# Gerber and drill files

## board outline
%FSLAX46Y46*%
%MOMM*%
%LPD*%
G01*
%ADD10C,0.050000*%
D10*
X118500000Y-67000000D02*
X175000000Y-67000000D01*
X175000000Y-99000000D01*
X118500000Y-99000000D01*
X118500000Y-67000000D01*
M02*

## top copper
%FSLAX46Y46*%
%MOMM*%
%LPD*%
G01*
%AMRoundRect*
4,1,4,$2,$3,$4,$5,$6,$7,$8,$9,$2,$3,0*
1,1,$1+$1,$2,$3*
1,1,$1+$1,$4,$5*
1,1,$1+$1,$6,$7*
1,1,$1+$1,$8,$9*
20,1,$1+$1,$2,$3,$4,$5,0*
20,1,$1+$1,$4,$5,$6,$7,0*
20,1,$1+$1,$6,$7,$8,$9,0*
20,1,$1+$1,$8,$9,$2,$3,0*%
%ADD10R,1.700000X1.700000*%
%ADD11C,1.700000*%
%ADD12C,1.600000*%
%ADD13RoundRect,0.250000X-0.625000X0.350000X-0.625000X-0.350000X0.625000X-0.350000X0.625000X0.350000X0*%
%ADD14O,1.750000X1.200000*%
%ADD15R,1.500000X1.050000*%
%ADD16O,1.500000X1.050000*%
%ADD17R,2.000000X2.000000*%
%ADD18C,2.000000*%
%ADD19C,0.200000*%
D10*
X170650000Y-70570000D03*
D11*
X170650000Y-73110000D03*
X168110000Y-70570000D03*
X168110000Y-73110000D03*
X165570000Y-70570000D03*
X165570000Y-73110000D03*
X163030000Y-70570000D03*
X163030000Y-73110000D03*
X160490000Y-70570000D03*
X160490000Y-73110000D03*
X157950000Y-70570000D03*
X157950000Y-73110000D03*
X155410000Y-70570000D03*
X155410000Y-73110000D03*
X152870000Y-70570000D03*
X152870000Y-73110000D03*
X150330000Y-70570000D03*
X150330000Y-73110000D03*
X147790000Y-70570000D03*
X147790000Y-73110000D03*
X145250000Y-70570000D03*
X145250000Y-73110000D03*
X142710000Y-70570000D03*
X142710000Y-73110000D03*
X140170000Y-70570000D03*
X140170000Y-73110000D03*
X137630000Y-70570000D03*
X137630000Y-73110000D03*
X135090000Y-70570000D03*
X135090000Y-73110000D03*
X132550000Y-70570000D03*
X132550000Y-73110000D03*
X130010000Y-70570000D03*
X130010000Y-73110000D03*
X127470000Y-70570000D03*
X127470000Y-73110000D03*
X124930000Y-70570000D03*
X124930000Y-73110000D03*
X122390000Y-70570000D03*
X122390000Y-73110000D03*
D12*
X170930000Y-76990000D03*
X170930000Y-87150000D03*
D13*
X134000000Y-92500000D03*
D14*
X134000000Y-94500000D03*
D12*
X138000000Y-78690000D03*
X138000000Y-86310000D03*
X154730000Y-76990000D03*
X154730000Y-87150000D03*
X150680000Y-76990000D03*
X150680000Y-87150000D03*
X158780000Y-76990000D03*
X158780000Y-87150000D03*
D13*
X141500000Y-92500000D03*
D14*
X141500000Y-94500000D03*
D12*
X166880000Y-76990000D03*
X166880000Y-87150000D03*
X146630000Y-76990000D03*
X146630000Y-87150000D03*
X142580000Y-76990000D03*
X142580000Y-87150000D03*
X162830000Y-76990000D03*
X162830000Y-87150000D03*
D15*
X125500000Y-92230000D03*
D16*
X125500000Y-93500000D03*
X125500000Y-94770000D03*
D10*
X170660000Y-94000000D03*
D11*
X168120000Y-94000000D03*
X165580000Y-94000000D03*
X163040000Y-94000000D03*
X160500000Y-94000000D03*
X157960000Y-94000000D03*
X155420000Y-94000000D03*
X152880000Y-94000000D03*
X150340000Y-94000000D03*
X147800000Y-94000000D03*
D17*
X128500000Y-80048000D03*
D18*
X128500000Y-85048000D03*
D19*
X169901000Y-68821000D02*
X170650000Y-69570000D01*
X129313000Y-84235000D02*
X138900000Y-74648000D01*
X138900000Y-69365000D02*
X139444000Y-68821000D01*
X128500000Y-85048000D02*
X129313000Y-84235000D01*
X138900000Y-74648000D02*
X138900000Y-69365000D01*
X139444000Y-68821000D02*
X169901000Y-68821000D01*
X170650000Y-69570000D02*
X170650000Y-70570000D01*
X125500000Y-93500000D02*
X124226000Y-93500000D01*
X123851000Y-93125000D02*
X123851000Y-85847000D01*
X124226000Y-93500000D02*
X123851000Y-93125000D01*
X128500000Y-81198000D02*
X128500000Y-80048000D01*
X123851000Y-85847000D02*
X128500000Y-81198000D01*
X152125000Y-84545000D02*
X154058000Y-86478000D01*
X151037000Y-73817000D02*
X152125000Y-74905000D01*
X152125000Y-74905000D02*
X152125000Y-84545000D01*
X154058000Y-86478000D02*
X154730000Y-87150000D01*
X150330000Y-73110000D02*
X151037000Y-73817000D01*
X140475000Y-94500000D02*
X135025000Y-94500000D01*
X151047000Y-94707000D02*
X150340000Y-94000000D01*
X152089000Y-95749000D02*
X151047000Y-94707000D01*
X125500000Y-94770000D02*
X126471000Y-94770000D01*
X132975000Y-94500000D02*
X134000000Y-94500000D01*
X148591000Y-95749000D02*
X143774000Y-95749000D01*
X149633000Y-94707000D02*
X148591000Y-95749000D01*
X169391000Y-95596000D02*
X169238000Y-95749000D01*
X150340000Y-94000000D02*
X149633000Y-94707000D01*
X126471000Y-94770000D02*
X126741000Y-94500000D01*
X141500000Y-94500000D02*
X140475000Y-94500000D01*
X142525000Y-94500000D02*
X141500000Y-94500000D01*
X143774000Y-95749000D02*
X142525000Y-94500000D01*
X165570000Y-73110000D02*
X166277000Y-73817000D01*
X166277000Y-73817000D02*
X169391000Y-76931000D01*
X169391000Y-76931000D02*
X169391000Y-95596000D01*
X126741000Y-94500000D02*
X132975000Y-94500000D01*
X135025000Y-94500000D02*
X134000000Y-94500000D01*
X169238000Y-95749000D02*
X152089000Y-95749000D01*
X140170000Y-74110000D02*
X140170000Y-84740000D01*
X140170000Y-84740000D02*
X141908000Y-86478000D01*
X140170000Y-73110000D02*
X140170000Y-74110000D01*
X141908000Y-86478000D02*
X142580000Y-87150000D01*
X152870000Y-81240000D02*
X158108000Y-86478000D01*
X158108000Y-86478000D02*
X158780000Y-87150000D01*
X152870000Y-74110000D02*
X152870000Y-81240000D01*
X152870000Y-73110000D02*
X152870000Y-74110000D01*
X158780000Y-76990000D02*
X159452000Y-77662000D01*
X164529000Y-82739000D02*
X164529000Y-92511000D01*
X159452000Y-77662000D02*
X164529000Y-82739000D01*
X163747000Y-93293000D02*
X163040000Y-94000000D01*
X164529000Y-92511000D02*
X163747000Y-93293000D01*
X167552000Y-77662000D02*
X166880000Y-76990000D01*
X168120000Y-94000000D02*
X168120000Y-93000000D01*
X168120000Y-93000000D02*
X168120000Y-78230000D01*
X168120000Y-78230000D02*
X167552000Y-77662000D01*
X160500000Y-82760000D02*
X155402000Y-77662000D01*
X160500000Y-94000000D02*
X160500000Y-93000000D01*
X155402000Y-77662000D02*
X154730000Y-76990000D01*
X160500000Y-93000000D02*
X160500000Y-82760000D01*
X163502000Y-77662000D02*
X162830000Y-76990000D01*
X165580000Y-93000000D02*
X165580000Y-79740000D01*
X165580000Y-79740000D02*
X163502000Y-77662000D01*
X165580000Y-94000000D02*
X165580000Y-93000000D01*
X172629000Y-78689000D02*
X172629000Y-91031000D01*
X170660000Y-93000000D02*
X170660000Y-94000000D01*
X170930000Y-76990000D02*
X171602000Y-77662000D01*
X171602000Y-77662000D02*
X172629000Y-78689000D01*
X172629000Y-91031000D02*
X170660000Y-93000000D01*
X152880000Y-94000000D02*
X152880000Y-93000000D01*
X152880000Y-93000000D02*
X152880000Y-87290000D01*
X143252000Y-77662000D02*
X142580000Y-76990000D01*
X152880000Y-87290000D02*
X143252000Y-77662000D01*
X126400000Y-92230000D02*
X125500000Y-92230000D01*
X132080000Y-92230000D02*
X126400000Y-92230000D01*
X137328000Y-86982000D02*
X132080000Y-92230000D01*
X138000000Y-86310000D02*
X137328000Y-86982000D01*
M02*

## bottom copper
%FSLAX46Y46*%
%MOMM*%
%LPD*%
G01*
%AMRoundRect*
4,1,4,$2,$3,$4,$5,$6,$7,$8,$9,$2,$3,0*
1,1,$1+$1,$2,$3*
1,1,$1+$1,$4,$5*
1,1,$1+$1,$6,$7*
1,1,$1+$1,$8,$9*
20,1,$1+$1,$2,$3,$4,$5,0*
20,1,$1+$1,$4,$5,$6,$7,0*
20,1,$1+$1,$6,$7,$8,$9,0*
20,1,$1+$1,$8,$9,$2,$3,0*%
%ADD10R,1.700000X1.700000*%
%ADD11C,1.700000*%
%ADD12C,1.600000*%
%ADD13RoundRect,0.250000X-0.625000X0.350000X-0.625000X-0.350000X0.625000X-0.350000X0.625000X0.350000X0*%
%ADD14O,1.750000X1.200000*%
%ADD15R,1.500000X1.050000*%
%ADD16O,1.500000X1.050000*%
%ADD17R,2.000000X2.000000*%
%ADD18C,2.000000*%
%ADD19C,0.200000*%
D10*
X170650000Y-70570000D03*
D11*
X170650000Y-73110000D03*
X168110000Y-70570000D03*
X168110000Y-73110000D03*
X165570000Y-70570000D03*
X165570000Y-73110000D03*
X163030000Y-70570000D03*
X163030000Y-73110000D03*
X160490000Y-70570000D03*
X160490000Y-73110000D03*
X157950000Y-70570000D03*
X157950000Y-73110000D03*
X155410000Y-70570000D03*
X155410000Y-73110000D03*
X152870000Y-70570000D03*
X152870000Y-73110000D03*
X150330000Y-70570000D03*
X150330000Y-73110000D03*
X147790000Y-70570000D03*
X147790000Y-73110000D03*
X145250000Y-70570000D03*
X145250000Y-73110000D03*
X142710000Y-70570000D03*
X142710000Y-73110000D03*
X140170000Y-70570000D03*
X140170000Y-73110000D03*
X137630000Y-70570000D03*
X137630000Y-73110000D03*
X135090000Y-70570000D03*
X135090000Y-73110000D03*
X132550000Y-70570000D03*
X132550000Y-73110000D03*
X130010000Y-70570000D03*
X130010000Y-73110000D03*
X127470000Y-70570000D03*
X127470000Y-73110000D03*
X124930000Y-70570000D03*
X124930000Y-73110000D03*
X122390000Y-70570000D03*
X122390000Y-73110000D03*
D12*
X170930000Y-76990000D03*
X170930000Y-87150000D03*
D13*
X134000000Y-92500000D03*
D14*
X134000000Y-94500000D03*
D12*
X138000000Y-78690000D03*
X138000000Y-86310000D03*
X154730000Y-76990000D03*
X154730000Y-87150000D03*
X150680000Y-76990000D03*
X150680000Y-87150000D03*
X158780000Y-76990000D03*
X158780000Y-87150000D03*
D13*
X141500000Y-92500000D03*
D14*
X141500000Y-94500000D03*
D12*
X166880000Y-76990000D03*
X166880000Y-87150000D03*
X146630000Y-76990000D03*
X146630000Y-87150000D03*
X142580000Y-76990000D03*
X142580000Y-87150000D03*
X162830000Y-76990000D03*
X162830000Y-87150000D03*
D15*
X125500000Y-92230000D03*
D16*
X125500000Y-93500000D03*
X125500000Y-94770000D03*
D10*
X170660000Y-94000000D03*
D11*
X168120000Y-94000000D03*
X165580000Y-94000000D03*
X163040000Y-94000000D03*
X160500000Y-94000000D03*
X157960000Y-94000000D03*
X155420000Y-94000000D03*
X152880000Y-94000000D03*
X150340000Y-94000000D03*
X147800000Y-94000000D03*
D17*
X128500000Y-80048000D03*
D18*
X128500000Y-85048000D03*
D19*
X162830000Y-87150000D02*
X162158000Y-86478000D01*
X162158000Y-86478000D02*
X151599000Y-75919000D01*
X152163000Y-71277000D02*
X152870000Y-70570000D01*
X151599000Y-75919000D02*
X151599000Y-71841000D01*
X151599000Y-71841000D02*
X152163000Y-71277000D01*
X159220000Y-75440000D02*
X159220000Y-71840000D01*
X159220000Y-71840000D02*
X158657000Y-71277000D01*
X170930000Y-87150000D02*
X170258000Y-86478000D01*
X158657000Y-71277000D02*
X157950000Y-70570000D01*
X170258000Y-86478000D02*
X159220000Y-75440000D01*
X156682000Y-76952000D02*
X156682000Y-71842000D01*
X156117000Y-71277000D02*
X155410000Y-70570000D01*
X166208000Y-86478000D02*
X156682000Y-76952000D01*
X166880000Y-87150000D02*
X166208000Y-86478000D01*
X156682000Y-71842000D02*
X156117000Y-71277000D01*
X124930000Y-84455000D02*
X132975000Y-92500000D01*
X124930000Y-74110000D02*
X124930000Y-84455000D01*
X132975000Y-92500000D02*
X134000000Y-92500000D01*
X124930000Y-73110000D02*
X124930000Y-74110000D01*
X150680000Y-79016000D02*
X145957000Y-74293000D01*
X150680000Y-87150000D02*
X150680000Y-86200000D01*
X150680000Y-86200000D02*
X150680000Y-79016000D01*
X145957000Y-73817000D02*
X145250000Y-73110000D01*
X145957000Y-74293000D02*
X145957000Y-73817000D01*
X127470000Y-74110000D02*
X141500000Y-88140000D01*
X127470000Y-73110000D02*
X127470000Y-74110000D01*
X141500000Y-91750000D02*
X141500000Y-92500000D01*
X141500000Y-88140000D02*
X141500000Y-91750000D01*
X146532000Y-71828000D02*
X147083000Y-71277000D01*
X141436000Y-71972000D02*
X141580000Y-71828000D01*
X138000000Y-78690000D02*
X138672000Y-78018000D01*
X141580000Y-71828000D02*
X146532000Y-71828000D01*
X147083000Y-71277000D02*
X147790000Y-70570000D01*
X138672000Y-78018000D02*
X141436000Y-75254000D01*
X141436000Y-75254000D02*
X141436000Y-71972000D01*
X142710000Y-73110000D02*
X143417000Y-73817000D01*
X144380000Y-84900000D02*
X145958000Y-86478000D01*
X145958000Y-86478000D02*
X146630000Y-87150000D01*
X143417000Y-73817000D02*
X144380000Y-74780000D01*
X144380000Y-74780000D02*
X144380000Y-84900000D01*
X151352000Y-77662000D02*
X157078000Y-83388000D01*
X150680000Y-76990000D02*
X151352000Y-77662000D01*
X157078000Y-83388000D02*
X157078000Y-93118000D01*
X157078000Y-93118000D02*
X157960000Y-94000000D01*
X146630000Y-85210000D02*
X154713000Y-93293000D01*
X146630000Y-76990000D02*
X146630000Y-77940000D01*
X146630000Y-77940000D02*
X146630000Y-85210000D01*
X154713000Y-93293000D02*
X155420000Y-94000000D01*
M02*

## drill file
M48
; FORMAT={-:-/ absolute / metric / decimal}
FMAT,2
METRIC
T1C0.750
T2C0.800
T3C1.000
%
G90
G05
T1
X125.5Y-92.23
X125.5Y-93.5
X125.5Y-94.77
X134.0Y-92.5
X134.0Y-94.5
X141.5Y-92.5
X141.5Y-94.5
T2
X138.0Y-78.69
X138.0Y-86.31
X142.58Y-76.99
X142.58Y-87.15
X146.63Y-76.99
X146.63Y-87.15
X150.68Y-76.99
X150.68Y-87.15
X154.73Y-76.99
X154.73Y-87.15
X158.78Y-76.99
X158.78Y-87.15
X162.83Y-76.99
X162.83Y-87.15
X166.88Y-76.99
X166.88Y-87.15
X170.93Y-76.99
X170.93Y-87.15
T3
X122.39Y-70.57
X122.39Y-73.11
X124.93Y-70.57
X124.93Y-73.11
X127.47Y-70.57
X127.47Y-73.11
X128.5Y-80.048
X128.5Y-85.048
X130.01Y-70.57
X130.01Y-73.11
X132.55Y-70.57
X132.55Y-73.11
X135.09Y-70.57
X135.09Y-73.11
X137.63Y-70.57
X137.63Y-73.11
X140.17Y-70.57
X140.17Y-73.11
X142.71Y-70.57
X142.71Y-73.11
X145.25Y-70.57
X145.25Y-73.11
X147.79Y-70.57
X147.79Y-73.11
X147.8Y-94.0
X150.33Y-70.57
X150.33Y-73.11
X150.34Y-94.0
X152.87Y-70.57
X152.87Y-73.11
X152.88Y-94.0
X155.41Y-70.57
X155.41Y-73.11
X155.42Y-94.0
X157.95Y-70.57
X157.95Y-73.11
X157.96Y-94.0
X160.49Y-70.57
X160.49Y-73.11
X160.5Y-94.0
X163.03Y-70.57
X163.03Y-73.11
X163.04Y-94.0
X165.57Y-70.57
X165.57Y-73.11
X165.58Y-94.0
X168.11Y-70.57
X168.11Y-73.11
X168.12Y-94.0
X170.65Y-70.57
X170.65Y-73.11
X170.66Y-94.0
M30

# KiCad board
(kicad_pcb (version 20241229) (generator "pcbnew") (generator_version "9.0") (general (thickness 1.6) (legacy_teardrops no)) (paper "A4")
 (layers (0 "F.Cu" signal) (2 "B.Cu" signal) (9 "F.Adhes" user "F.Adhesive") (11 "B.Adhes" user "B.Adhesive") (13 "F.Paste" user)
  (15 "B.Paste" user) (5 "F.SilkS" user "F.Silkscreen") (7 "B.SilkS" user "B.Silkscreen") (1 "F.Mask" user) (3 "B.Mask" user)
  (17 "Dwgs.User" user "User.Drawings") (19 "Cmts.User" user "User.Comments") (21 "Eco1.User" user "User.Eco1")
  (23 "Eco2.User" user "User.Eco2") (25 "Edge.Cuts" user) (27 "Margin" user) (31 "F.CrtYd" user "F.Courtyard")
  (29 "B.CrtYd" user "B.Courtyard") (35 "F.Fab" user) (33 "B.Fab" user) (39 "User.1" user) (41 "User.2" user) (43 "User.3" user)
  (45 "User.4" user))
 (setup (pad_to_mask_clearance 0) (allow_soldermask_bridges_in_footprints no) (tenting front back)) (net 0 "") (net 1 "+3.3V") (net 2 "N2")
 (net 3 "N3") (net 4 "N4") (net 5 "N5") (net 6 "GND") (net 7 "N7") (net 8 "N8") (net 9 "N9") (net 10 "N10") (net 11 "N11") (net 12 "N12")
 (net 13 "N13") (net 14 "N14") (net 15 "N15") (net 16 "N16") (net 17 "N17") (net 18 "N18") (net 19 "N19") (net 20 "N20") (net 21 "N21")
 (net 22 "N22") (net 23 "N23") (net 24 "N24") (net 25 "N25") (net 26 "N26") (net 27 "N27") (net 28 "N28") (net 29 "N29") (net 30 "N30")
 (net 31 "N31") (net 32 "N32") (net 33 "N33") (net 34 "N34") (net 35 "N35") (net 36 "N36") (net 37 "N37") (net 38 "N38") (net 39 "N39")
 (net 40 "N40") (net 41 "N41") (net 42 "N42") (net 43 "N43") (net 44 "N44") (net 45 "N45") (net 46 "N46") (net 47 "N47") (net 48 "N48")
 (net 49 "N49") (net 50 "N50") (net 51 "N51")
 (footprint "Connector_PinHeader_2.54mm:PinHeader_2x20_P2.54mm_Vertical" (layer "F.Cu") (at 170.65 70.57 -90)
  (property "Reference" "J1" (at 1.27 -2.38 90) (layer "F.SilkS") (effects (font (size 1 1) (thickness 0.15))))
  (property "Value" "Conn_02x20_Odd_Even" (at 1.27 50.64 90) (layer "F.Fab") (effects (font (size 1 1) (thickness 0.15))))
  (pad "1" thru_hole rect (at 0 0 270) (size 1.7 1.7) (drill 1) (layers "*.Cu" "*.Mask") (remove_unused_layers no) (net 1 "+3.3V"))
  (pad "2" thru_hole circle (at 2.54 0 270) (size 1.7 1.7) (drill 1) (layers "*.Cu" "*.Mask") (remove_unused_layers no) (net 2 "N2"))
  (pad "3" thru_hole circle (at 0 2.54 270) (size 1.7 1.7) (drill 1) (layers "*.Cu" "*.Mask") (remove_unused_layers no) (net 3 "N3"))
  (pad "4" thru_hole circle (at 2.54 2.54 270) (size 1.7 1.7) (drill 1) (layers "*.Cu" "*.Mask") (remove_unused_layers no) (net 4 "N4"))
  (pad "5" thru_hole circle (at 0 5.08 270) (size 1.7 1.7) (drill 1) (layers "*.Cu" "*.Mask") (remove_unused_layers no) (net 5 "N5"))
  (pad "6" thru_hole circle (at 2.54 5.08 270) (size 1.7 1.7) (drill 1) (layers "*.Cu" "*.Mask") (remove_unused_layers no) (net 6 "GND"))
  (pad "7" thru_hole circle (at 0 7.62 270) (size 1.7 1.7) (drill 1) (layers "*.Cu" "*.Mask") (remove_unused_layers no) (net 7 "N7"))
  (pad "8" thru_hole circle (at 2.54 7.62 270) (size 1.7 1.7) (drill 1) (layers "*.Cu" "*.Mask") (remove_unused_layers no) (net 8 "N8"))
  (pad "9" thru_hole circle (at 0 10.16 270) (size 1.7 1.7) (drill 1) (layers "*.Cu" "*.Mask") (remove_unused_layers no) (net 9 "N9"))
  (pad "10" thru_hole circle (at 2.54 10.16 270) (size 1.7 1.7) (drill 1) (layers "*.Cu" "*.Mask") (remove_unused_layers no) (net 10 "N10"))
  (pad "11" thru_hole circle (at 0 12.7 270) (size 1.7 1.7) (drill 1) (layers "*.Cu" "*.Mask") (remove_unused_layers no) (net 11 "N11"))
  (pad "12" thru_hole circle (at 2.54 12.7 270) (size 1.7 1.7) (drill 1) (layers "*.Cu" "*.Mask") (remove_unused_layers no) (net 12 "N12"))
  (pad "13" thru_hole circle (at 0 15.24 270) (size 1.7 1.7) (drill 1) (layers "*.Cu" "*.Mask") (remove_unused_layers no) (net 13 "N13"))
  (pad "14" thru_hole circle (at 2.54 15.24 270) (size 1.7 1.7) (drill 1) (layers "*.Cu" "*.Mask") (remove_unused_layers no) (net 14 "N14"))
  (pad "15" thru_hole circle (at 0 17.78 270) (size 1.7 1.7) (drill 1) (layers "*.Cu" "*.Mask") (remove_unused_layers no) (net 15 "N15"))
  (pad "16" thru_hole circle (at 2.54 17.78 270) (size 1.7 1.7) (drill 1) (layers "*.Cu" "*.Mask") (remove_unused_layers no) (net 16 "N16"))
  (pad "17" thru_hole circle (at 0 20.32 270) (size 1.7 1.7) (drill 1) (layers "*.Cu" "*.Mask") (remove_unused_layers no) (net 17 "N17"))
  (pad "18" thru_hole circle (at 2.54 20.32 270) (size 1.7 1.7) (drill 1) (layers "*.Cu" "*.Mask") (remove_unused_layers no) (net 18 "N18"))
  (pad "19" thru_hole circle (at 0 22.86 270) (size 1.7 1.7) (drill 1) (layers "*.Cu" "*.Mask") (remove_unused_layers no) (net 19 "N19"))
  (pad "20" thru_hole circle (at 2.54 22.86 270) (size 1.7 1.7) (drill 1) (layers "*.Cu" "*.Mask") (remove_unused_layers no) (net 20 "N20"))
  (pad "21" thru_hole circle (at 0 25.4 270) (size 1.7 1.7) (drill 1) (layers "*.Cu" "*.Mask") (remove_unused_layers no) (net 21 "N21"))
  (pad "22" thru_hole circle (at 2.54 25.4 270) (size 1.7 1.7) (drill 1) (layers "*.Cu" "*.Mask") (remove_unused_layers no) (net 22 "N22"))
  (pad "23" thru_hole circle (at 0 27.94 270) (size 1.7 1.7) (drill 1) (layers "*.Cu" "*.Mask") (remove_unused_layers no) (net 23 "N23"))
  (pad "24" thru_hole circle (at 2.54 27.94 270) (size 1.7 1.7) (drill 1) (layers "*.Cu" "*.Mask") (remove_unused_layers no) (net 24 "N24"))
  (pad "25" thru_hole circle (at 0 30.48 270) (size 1.7 1.7) (drill 1) (layers "*.Cu" "*.Mask") (remove_unused_layers no) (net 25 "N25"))
  (pad "26" thru_hole circle (at 2.54 30.48 270) (size 1.7 1.7) (drill 1) (layers "*.Cu" "*.Mask") (remove_unused_layers no) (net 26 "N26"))
  (pad "27" thru_hole circle (at 0 33.02 270) (size 1.7 1.7) (drill 1) (layers "*.Cu" "*.Mask") (remove_unused_layers no) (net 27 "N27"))
  (pad "28" thru_hole circle (at 2.54 33.02 270) (size 1.7 1.7) (drill 1) (layers "*.Cu" "*.Mask") (remove_unused_layers no) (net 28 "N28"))
  (pad "29" thru_hole circle (at 0 35.56 270) (size 1.7 1.7) (drill 1) (layers "*.Cu" "*.Mask") (remove_unused_layers no) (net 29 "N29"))
  (pad "30" thru_hole circle (at 2.54 35.56 270) (size 1.7 1.7) (drill 1) (layers "*.Cu" "*.Mask") (remove_unused_layers no) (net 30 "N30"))
  (pad "31" thru_hole circle (at 0 38.1 270) (size 1.7 1.7) (drill 1) (layers "*.Cu" "*.Mask") (remove_unused_layers no) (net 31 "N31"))
  (pad "32" thru_hole circle (at 2.54 38.1 270) (size 1.7 1.7) (drill 1) (layers "*.Cu" "*.Mask") (remove_unused_layers no) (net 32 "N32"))
  (pad "33" thru_hole circle (at 0 40.64 270) (size 1.7 1.7) (drill 1) (layers "*.Cu" "*.Mask") (remove_unused_layers no) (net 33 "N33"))
  (pad "34" thru_hole circle (at 2.54 40.64 270) (size 1.7 1.7) (drill 1) (layers "*.Cu" "*.Mask") (remove_unused_layers no) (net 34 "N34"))
  (pad "35" thru_hole circle (at 0 43.18 270) (size 1.7 1.7) (drill 1) (layers "*.Cu" "*.Mask") (remove_unused_layers no) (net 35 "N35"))
  (pad "36" thru_hole circle (at 2.54 43.18 270) (size 1.7 1.7) (drill 1) (layers "*.Cu" "*.Mask") (remove_unused_layers no) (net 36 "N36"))
  (pad "37" thru_hole circle (at 0 45.72 270) (size 1.7 1.7) (drill 1) (layers "*.Cu" "*.Mask") (remove_unused_layers no) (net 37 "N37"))
  (pad "38" thru_hole circle (at 2.54 45.72 270) (size 1.7 1.7) (drill 1) (layers "*.Cu" "*.Mask") (remove_unused_layers no) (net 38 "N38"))
  (pad "39" thru_hole circle (at 0 48.26 270) (size 1.7 1.7) (drill 1) (layers "*.Cu" "*.Mask") (remove_unused_layers no) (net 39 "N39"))
  (pad "40" thru_hole circle (at 2.54 48.26 270) (size 1.7 1.7) (drill 1) (layers "*.Cu" "*.Mask") (remove_unused_layers no) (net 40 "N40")))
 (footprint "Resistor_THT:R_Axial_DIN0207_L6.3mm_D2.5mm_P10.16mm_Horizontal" (layer "F.Cu") (at 170.93 76.99 -90)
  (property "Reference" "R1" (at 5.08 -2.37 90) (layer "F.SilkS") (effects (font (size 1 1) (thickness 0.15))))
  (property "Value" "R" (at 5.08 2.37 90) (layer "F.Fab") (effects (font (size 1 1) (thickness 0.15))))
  (pad "1" thru_hole circle (at 0 0 270) (size 1.6 1.6) (drill 0.8) (layers "*.Cu" "*.Mask") (remove_unused_layers no) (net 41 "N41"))
  (pad "2" thru_hole circle (at 10.16 0 270) (size 1.6 1.6) (drill 0.8) (layers "*.Cu" "*.Mask") (remove_unused_layers no) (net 11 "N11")))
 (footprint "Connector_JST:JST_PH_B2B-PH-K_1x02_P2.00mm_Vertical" (layer "F.Cu") (at 134 92.5 -90)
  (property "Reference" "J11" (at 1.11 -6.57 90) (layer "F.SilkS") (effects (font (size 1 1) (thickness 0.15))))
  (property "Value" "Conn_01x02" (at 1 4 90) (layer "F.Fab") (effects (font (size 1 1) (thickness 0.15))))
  (pad "1" thru_hole roundrect (at 0 0 270) (size 1.2 1.75) (drill 0.75) (layers "*.Cu" "*.Mask") (remove_unused_layers no)
   (roundrect_rratio 0.208333) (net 38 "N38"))
  (pad "2" thru_hole oval (at 2 0 270) (size 1.2 1.75) (drill 0.75) (layers "*.Cu" "*.Mask") (remove_unused_layers no) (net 6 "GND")))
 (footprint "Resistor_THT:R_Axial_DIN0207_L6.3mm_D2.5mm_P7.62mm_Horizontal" (layer "F.Cu") (at 138 78.69 -90)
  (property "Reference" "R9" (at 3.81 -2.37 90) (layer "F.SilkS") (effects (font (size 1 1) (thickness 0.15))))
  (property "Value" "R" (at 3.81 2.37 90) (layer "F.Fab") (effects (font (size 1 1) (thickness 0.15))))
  (pad "1" thru_hole circle (at 0 0 270) (size 1.6 1.6) (drill 0.8) (layers "*.Cu" "*.Mask") (remove_unused_layers no) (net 19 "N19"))
  (pad "2" thru_hole circle (at 7.62 0 270) (size 1.6 1.6) (drill 0.8) (layers "*.Cu" "*.Mask") (remove_unused_layers no) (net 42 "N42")))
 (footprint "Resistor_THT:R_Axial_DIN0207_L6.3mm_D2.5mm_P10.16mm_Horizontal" (layer "F.Cu") (at 154.73 76.99 -90)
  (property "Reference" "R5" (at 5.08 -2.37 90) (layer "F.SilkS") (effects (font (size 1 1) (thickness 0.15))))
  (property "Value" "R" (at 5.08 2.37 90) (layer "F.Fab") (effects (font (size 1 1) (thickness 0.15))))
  (pad "1" thru_hole circle (at 0 0 270) (size 1.6 1.6) (drill 0.8) (layers "*.Cu" "*.Mask") (remove_unused_layers no) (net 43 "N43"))
  (pad "2" thru_hole circle (at 10.16 0 270) (size 1.6 1.6) (drill 0.8) (layers "*.Cu" "*.Mask") (remove_unused_layers no) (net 18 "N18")))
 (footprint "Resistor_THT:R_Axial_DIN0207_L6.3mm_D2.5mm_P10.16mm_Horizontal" (layer "F.Cu") (at 150.68 76.99 -90)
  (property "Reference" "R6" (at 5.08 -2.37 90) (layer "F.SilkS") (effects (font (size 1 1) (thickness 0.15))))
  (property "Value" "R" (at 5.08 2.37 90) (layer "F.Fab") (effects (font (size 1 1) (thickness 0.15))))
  (pad "1" thru_hole circle (at 0 0 270) (size 1.6 1.6) (drill 0.8) (layers "*.Cu" "*.Mask") (remove_unused_layers no) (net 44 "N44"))
  (pad "2" thru_hole circle (at 10.16 0 270) (size 1.6 1.6) (drill 0.8) (layers "*.Cu" "*.Mask") (remove_unused_layers no) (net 22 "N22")))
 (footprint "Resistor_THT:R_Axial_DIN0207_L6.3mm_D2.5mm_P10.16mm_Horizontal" (layer "F.Cu") (at 158.78 76.99 -90)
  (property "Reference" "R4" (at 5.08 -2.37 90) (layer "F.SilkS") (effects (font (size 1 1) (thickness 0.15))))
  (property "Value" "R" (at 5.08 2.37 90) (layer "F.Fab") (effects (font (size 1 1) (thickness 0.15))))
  (pad "1" thru_hole circle (at 0 0 270) (size 1.6 1.6) (drill 0.8) (layers "*.Cu" "*.Mask") (remove_unused_layers no) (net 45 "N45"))
  (pad "2" thru_hole circle (at 10.16 0 270) (size 1.6 1.6) (drill 0.8) (layers "*.Cu" "*.Mask") (remove_unused_layers no) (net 16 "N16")))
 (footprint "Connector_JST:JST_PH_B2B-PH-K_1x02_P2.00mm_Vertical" (layer "F.Cu") (at 141.5 92.5 -90)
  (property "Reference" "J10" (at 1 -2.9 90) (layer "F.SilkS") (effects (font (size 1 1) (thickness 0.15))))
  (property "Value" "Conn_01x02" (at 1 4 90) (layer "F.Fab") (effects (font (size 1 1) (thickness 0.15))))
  (pad "1" thru_hole roundrect (at 0 0 270) (size 1.2 1.75) (drill 0.75) (layers "*.Cu" "*.Mask") (remove_unused_layers no)
   (roundrect_rratio 0.208333) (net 36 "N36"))
  (pad "2" thru_hole oval (at 2 0 270) (size 1.2 1.75) (drill 0.75) (layers "*.Cu" "*.Mask") (remove_unused_layers no) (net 6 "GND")))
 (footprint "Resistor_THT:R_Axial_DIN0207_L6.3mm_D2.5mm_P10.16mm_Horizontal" (layer "F.Cu") (at 166.88 76.99 -90)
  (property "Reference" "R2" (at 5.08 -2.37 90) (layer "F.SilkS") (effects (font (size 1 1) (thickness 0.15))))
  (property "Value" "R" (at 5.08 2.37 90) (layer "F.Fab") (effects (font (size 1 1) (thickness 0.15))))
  (pad "1" thru_hole circle (at 0 0 270) (size 1.6 1.6) (drill 0.8) (layers "*.Cu" "*.Mask") (remove_unused_layers no) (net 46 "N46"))
  (pad "2" thru_hole circle (at 10.16 0 270) (size 1.6 1.6) (drill 0.8) (layers "*.Cu" "*.Mask") (remove_unused_layers no) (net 13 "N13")))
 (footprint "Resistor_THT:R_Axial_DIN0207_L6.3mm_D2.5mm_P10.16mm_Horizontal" (layer "F.Cu") (at 146.63 76.99 -90)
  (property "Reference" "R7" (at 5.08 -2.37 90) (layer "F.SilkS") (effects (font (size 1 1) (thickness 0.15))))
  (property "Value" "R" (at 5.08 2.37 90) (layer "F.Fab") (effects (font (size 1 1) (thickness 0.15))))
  (pad "1" thru_hole circle (at 0 0 270) (size 1.6 1.6) (drill 0.8) (layers "*.Cu" "*.Mask") (remove_unused_layers no) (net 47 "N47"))
  (pad "2" thru_hole circle (at 10.16 0 270) (size 1.6 1.6) (drill 0.8) (layers "*.Cu" "*.Mask") (remove_unused_layers no) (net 24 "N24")))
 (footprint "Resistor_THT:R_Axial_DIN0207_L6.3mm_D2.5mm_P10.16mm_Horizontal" (layer "F.Cu") (at 142.58 76.99 -90)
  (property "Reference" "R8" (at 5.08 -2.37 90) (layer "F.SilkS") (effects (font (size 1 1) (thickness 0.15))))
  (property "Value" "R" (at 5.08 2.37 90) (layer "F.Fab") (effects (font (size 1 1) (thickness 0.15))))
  (pad "1" thru_hole circle (at 0 0 270) (size 1.6 1.6) (drill 0.8) (layers "*.Cu" "*.Mask") (remove_unused_layers no) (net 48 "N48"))
  (pad "2" thru_hole circle (at 10.16 0 270) (size 1.6 1.6) (drill 0.8) (layers "*.Cu" "*.Mask") (remove_unused_layers no) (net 26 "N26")))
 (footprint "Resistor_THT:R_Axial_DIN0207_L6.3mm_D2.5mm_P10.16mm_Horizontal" (layer "F.Cu") (at 162.83 76.99 -90)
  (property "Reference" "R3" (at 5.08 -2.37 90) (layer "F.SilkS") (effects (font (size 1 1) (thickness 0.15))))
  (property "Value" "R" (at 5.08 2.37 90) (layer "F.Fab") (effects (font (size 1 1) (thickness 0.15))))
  (pad "1" thru_hole circle (at 0 0 270) (size 1.6 1.6) (drill 0.8) (layers "*.Cu" "*.Mask") (remove_unused_layers no) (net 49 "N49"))
  (pad "2" thru_hole circle (at 10.16 0 270) (size 1.6 1.6) (drill 0.8) (layers "*.Cu" "*.Mask") (remove_unused_layers no) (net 15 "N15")))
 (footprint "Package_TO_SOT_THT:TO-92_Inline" (layer "F.Cu") (at 125.5 92.23 -90)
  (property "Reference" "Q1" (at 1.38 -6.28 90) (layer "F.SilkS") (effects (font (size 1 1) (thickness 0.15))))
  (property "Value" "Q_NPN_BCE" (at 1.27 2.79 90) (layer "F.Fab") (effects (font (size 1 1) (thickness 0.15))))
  (pad "1" thru_hole rect (at 0 0 270) (size 1.05 1.5) (drill 0.75) (layers "*.Cu" "*.Mask") (remove_unused_layers no) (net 42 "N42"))
  (pad "2" thru_hole oval (at 1.27 0 270) (size 1.05 1.5) (drill 0.75) (layers "*.Cu" "*.Mask") (remove_unused_layers no) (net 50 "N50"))
  (pad "3" thru_hole oval (at 2.54 0 270) (size 1.05 1.5) (drill 0.75) (layers "*.Cu" "*.Mask") (remove_unused_layers no) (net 6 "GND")))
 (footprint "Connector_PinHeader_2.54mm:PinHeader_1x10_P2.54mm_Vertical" (layer "F.Cu") (at 170.66 94 -90)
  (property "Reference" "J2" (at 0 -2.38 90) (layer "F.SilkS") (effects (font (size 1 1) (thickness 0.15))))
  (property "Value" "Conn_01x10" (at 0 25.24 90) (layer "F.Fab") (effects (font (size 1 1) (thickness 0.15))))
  (pad "1" thru_hole rect (at 0 0 270) (size 1.7 1.7) (drill 1) (layers "*.Cu" "*.Mask") (remove_unused_layers no) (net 41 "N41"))
  (pad "2" thru_hole circle (at 0 2.54 270) (size 1.7 1.7) (drill 1) (layers "*.Cu" "*.Mask") (remove_unused_layers no) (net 46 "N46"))
  (pad "3" thru_hole circle (at 0 5.08 270) (size 1.7 1.7) (drill 1) (layers "*.Cu" "*.Mask") (remove_unused_layers no) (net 49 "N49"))
  (pad "4" thru_hole circle (at 0 7.62 270) (size 1.7 1.7) (drill 1) (layers "*.Cu" "*.Mask") (remove_unused_layers no) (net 45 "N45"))
  (pad "5" thru_hole circle (at 0 10.16 270) (size 1.7 1.7) (drill 1) (layers "*.Cu" "*.Mask") (remove_unused_layers no) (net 43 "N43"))
  (pad "6" thru_hole circle (at 0 12.7 270) (size 1.7 1.7) (drill 1) (layers "*.Cu" "*.Mask") (remove_unused_layers no) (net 44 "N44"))
  (pad "7" thru_hole circle (at 0 15.24 270) (size 1.7 1.7) (drill 1) (layers "*.Cu" "*.Mask") (remove_unused_layers no) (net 47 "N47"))
  (pad "8" thru_hole circle (at 0 17.78 270) (size 1.7 1.7) (drill 1) (layers "*.Cu" "*.Mask") (remove_unused_layers no) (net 48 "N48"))
  (pad "9" thru_hole circle (at 0 20.32 270) (size 1.7 1.7) (drill 1) (layers "*.Cu" "*.Mask") (remove_unused_layers no) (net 6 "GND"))
  (pad "10" thru_hole circle (at 0 22.86 270) (size 1.7 1.7) (drill 1) (layers "*.Cu" "*.Mask") (remove_unused_layers no) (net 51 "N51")))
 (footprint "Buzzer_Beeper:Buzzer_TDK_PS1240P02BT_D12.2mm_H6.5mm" (layer "F.Cu") (at 128.5 80.048 -90)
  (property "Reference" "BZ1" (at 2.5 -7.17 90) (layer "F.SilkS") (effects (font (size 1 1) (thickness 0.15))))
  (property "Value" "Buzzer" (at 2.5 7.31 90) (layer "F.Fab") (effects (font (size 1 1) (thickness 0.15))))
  (pad "1" thru_hole rect (at 0 0 270) (size 2 2) (drill 1) (layers "*.Cu" "*.Mask") (remove_unused_layers no) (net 50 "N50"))
  (pad "2" thru_hole circle (at 5 0 270) (size 2 2) (drill 1) (layers "*.Cu" "*.Mask") (remove_unused_layers no) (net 1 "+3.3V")))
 (gr_rect (start 118.5 67) (end 175 99) (stroke (width 0.05) (type default)) (fill no) (layer "Edge.Cuts"))
 (segment (start 169.901 68.821) (end 170.65 69.57) (width 0.2) (layer "F.Cu") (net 1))
 (segment (start 129.313 84.235) (end 138.9 74.648) (width 0.2) (layer "F.Cu") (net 1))
 (segment (start 138.9 69.365) (end 139.444 68.821) (width 0.2) (layer "F.Cu") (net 1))
 (segment (start 128.5 85.048) (end 129.313 84.235) (width 0.2) (layer "F.Cu") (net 1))
 (segment (start 138.9 74.648) (end 138.9 69.365) (width 0.2) (layer "F.Cu") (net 1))
 (segment (start 139.444 68.821) (end 169.901 68.821) (width 0.2) (layer "F.Cu") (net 1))
 (segment (start 170.65 69.57) (end 170.65 70.57) (width 0.2) (layer "F.Cu") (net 1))
 (segment (start 125.5 93.5) (end 124.226 93.5) (width 0.2) (layer "F.Cu") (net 50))
 (segment (start 123.851 93.125) (end 123.851 85.847) (width 0.2) (layer "F.Cu") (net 50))
 (segment (start 124.226 93.5) (end 123.851 93.125) (width 0.2) (layer "F.Cu") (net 50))
 (segment (start 128.5 81.198) (end 128.5 80.048) (width 0.2) (layer "F.Cu") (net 50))
 (segment (start 123.851 85.847) (end 128.5 81.198) (width 0.2) (layer "F.Cu") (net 50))
 (segment (start 152.125 84.545) (end 154.058 86.478) (width 0.2) (layer "F.Cu") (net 18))
 (segment (start 151.037 73.817) (end 152.125 74.905) (width 0.2) (layer "F.Cu") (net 18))
 (segment (start 152.125 74.905) (end 152.125 84.545) (width 0.2) (layer "F.Cu") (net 18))
 (segment (start 154.058 86.478) (end 154.73 87.15) (width 0.2) (layer "F.Cu") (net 18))
 (segment (start 150.33 73.11) (end 151.037 73.817) (width 0.2) (layer "F.Cu") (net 18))
 (segment (start 162.83 87.15) (end 162.158 86.478) (width 0.2) (layer "B.Cu") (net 15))
 (segment (start 162.158 86.478) (end 151.599 75.919) (width 0.2) (layer "B.Cu") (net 15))
 (segment (start 152.163 71.277) (end 152.87 70.57) (width 0.2) (layer "B.Cu") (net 15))
 (segment (start 151.599 75.919) (end 151.599 71.841) (width 0.2) (layer "B.Cu") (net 15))
 (segment (start 151.599 71.841) (end 152.163 71.277) (width 0.2) (layer "B.Cu") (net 15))
 (segment (start 159.22 75.44) (end 159.22 71.84) (width 0.2) (layer "B.Cu") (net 11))
 (segment (start 159.22 71.84) (end 158.657 71.277) (width 0.2) (layer "B.Cu") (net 11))
 (segment (start 170.93 87.15) (end 170.258 86.478) (width 0.2) (layer "B.Cu") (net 11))
 (segment (start 158.657 71.277) (end 157.95 70.57) (width 0.2) (layer "B.Cu") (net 11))
 (segment (start 170.258 86.478) (end 159.22 75.44) (width 0.2) (layer "B.Cu") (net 11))
 (segment (start 156.682 76.952) (end 156.682 71.842) (width 0.2) (layer "B.Cu") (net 13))
 (segment (start 156.117 71.277) (end 155.41 70.57) (width 0.2) (layer "B.Cu") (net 13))
 (segment (start 166.208 86.478) (end 156.682 76.952) (width 0.2) (layer "B.Cu") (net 13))
 (segment (start 166.88 87.15) (end 166.208 86.478) (width 0.2) (layer "B.Cu") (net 13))
 (segment (start 156.682 71.842) (end 156.117 71.277) (width 0.2) (layer "B.Cu") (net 13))
 (segment (start 124.93 84.455) (end 132.975 92.5) (width 0.2) (layer "B.Cu") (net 38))
 (segment (start 124.93 74.11) (end 124.93 84.455) (width 0.2) (layer "B.Cu") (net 38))
 (segment (start 132.975 92.5) (end 134 92.5) (width 0.2) (layer "B.Cu") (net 38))
 (segment (start 124.93 73.11) (end 124.93 74.11) (width 0.2) (layer "B.Cu") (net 38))
 (segment (start 140.475 94.5) (end 135.025 94.5) (width 0.2) (layer "F.Cu") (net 6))
 (segment (start 151.047 94.707) (end 150.34 94) (width 0.2) (layer "F.Cu") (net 6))
 (segment (start 152.089 95.749) (end 151.047 94.707) (width 0.2) (layer "F.Cu") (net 6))
 (segment (start 125.5 94.77) (end 126.471 94.77) (width 0.2) (layer "F.Cu") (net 6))
 (segment (start 132.975 94.5) (end 134 94.5) (width 0.2) (layer "F.Cu") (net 6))
 (segment (start 148.591 95.749) (end 143.774 95.749) (width 0.2) (layer "F.Cu") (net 6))
 (segment (start 149.633 94.707) (end 148.591 95.749) (width 0.2) (layer "F.Cu") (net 6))
 (segment (start 169.391 95.596) (end 169.238 95.749) (width 0.2) (layer "F.Cu") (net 6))
 (segment (start 150.34 94) (end 149.633 94.707) (width 0.2) (layer "F.Cu") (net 6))
 (segment (start 126.471 94.77) (end 126.741 94.5) (width 0.2) (layer "F.Cu") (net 6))
 (segment (start 141.5 94.5) (end 140.475 94.5) (width 0.2) (layer "F.Cu") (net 6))
 (segment (start 142.525 94.5) (end 141.5 94.5) (width 0.2) (layer "F.Cu") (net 6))
 (segment (start 143.774 95.749) (end 142.525 94.5) (width 0.2) (layer "F.Cu") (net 6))
 (segment (start 165.57 73.11) (end 166.277 73.817) (width 0.2) (layer "F.Cu") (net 6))
 (segment (start 166.277 73.817) (end 169.391 76.931) (width 0.2) (layer "F.Cu") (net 6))
 (segment (start 169.391 76.931) (end 169.391 95.596) (width 0.2) (layer "F.Cu") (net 6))
 (segment (start 126.741 94.5) (end 132.975 94.5) (width 0.2) (layer "F.Cu") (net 6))
 (segment (start 135.025 94.5) (end 134 94.5) (width 0.2) (layer "F.Cu") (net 6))
 (segment (start 169.238 95.749) (end 152.089 95.749) (width 0.2) (layer "F.Cu") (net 6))
 (segment (start 150.68 79.016) (end 145.957 74.293) (width 0.2) (layer "B.Cu") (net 22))
 (segment (start 150.68 87.15) (end 150.68 86.2) (width 0.2) (layer "B.Cu") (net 22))
 (segment (start 150.68 86.2) (end 150.68 79.016) (width 0.2) (layer "B.Cu") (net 22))
 (segment (start 145.957 73.817) (end 145.25 73.11) (width 0.2) (layer "B.Cu") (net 22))
 (segment (start 145.957 74.293) (end 145.957 73.817) (width 0.2) (layer "B.Cu") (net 22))
 (segment (start 127.47 74.11) (end 141.5 88.14) (width 0.2) (layer "B.Cu") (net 36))
 (segment (start 127.47 73.11) (end 127.47 74.11) (width 0.2) (layer "B.Cu") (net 36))
 (segment (start 141.5 91.75) (end 141.5 92.5) (width 0.2) (layer "B.Cu") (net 36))
 (segment (start 141.5 88.14) (end 141.5 91.75) (width 0.2) (layer "B.Cu") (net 36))
 (segment (start 146.532 71.828) (end 147.083 71.277) (width 0.2) (layer "B.Cu") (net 19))
 (segment (start 141.436 71.972) (end 141.58 71.828) (width 0.2) (layer "B.Cu") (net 19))
 (segment (start 138 78.69) (end 138.672 78.018) (width 0.2) (layer "B.Cu") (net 19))
 (segment (start 141.58 71.828) (end 146.532 71.828) (width 0.2) (layer "B.Cu") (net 19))
 (segment (start 147.083 71.277) (end 147.79 70.57) (width 0.2) (layer "B.Cu") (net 19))
 (segment (start 138.672 78.018) (end 141.436 75.254) (width 0.2) (layer "B.Cu") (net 19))
 (segment (start 141.436 75.254) (end 141.436 71.972) (width 0.2) (layer "B.Cu") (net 19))
 (segment (start 142.71 73.11) (end 143.417 73.817) (width 0.2) (layer "B.Cu") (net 24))
 (segment (start 144.38 84.9) (end 145.958 86.478) (width 0.2) (layer "B.Cu") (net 24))
 (segment (start 145.958 86.478) (end 146.63 87.15) (width 0.2) (layer "B.Cu") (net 24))
 (segment (start 143.417 73.817) (end 144.38 74.78) (width 0.2) (layer "B.Cu") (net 24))
 (segment (start 144.38 74.78) (end 144.38 84.9) (width 0.2) (layer "B.Cu") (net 24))
 (segment (start 140.17 74.11) (end 140.17 84.74) (width 0.2) (layer "F.Cu") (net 26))
 (segment (start 140.17 84.74) (end 141.908 86.478) (width 0.2) (layer "F.Cu") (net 26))
 (segment (start 140.17 73.11) (end 140.17 74.11) (width 0.2) (layer "F.Cu") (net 26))
 (segment (start 141.908 86.478) (end 142.58 87.15) (width 0.2) (layer "F.Cu") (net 26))
 (segment (start 152.87 81.24) (end 158.108 86.478) (width 0.2) (layer "F.Cu") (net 16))
 (segment (start 158.108 86.478) (end 158.78 87.15) (width 0.2) (layer "F.Cu") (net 16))
 (segment (start 152.87 74.11) (end 152.87 81.24) (width 0.2) (layer "F.Cu") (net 16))
 (segment (start 152.87 73.11) (end 152.87 74.11) (width 0.2) (layer "F.Cu") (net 16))
 (segment (start 158.78 76.99) (end 159.452 77.662) (width 0.2) (layer "F.Cu") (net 45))
 (segment (start 164.529 82.739) (end 164.529 92.511) (width 0.2) (layer "F.Cu") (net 45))
 (segment (start 159.452 77.662) (end 164.529 82.739) (width 0.2) (layer "F.Cu") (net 45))
 (segment (start 163.747 93.293) (end 163.04 94) (width 0.2) (layer "F.Cu") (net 45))
 (segment (start 164.529 92.511) (end 163.747 93.293) (width 0.2) (layer "F.Cu") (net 45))
 (segment (start 151.352 77.662) (end 157.078 83.388) (width 0.2) (layer "B.Cu") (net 44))
 (segment (start 150.68 76.99) (end 151.352 77.662) (width 0.2) (layer "B.Cu") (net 44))
 (segment (start 157.078 83.388) (end 157.078 93.118) (width 0.2) (layer "B.Cu") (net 44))
 (segment (start 157.078 93.118) (end 157.96 94) (width 0.2) (layer "B.Cu") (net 44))
 (segment (start 167.552 77.662) (end 166.88 76.99) (width 0.2) (layer "F.Cu") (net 46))
 (segment (start 168.12 94) (end 168.12 93) (width 0.2) (layer "F.Cu") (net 46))
 (segment (start 168.12 93) (end 168.12 78.23) (width 0.2) (layer "F.Cu") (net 46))
 (segment (start 168.12 78.23) (end 167.552 77.662) (width 0.2) (layer "F.Cu") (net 46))
 (segment (start 160.5 82.76) (end 155.402 77.662) (width 0.2) (layer "F.Cu") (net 43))
 (segment (start 160.5 94) (end 160.5 93) (width 0.2) (layer "F.Cu") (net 43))
 (segment (start 155.402 77.662) (end 154.73 76.99) (width 0.2) (layer "F.Cu") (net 43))
 (segment (start 160.5 93) (end 160.5 82.76) (width 0.2) (layer "F.Cu") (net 43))
 (segment (start 163.502 77.662) (end 162.83 76.99) (width 0.2) (layer "F.Cu") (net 49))
 (segment (start 165.58 93) (end 165.58 79.74) (width 0.2) (layer "F.Cu") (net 49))
 (segment (start 165.58 79.74) (end 163.502 77.662) (width 0.2) (layer "F.Cu") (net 49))
 (segment (start 165.58 94) (end 165.58 93) (width 0.2) (layer "F.Cu") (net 49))
 (segment (start 146.63 85.21) (end 154.713 93.293) (width 0.2) (layer "B.Cu") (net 47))
 (segment (start 146.63 76.99) (end 146.63 77.94) (width 0.2) (layer "B.Cu") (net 47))
 (segment (start 146.63 77.94) (end 146.63 85.21) (width 0.2) (layer "B.Cu") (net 47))
 (segment (start 154.713 93.293) (end 155.42 94) (width 0.2) (layer "B.Cu") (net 47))
 (segment (start 172.629 78.689) (end 172.629 91.031) (width 0.2) (layer "F.Cu") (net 41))
 (segment (start 170.66 93) (end 170.66 94) (width 0.2) (layer "F.Cu") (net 41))
 (segment (start 170.93 76.99) (end 171.602 77.662) (width 0.2) (layer "F.Cu") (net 41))
 (segment (start 171.602 77.662) (end 172.629 78.689) (width 0.2) (layer "F.Cu") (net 41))
 (segment (start 172.629 91.031) (end 170.66 93) (width 0.2) (layer "F.Cu") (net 41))
 (segment (start 152.88 94) (end 152.88 93) (width 0.2) (layer "F.Cu") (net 48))
 (segment (start 152.88 93) (end 152.88 87.29) (width 0.2) (layer "F.Cu") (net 48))
 (segment (start 143.252 77.662) (end 142.58 76.99) (width 0.2) (layer "F.Cu") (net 48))
 (segment (start 152.88 87.29) (end 143.252 77.662) (width 0.2) (layer "F.Cu") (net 48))
 (segment (start 126.4 92.23) (end 125.5 92.23) (width 0.2) (layer "F.Cu") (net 42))
 (segment (start 132.08 92.23) (end 126.4 92.23) (width 0.2) (layer "F.Cu") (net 42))
 (segment (start 137.328 86.982) (end 132.08 92.23) (width 0.2) (layer "F.Cu") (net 42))
 (segment (start 138 86.31) (end 137.328 86.982) (width 0.2) (layer "F.Cu") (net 42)))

